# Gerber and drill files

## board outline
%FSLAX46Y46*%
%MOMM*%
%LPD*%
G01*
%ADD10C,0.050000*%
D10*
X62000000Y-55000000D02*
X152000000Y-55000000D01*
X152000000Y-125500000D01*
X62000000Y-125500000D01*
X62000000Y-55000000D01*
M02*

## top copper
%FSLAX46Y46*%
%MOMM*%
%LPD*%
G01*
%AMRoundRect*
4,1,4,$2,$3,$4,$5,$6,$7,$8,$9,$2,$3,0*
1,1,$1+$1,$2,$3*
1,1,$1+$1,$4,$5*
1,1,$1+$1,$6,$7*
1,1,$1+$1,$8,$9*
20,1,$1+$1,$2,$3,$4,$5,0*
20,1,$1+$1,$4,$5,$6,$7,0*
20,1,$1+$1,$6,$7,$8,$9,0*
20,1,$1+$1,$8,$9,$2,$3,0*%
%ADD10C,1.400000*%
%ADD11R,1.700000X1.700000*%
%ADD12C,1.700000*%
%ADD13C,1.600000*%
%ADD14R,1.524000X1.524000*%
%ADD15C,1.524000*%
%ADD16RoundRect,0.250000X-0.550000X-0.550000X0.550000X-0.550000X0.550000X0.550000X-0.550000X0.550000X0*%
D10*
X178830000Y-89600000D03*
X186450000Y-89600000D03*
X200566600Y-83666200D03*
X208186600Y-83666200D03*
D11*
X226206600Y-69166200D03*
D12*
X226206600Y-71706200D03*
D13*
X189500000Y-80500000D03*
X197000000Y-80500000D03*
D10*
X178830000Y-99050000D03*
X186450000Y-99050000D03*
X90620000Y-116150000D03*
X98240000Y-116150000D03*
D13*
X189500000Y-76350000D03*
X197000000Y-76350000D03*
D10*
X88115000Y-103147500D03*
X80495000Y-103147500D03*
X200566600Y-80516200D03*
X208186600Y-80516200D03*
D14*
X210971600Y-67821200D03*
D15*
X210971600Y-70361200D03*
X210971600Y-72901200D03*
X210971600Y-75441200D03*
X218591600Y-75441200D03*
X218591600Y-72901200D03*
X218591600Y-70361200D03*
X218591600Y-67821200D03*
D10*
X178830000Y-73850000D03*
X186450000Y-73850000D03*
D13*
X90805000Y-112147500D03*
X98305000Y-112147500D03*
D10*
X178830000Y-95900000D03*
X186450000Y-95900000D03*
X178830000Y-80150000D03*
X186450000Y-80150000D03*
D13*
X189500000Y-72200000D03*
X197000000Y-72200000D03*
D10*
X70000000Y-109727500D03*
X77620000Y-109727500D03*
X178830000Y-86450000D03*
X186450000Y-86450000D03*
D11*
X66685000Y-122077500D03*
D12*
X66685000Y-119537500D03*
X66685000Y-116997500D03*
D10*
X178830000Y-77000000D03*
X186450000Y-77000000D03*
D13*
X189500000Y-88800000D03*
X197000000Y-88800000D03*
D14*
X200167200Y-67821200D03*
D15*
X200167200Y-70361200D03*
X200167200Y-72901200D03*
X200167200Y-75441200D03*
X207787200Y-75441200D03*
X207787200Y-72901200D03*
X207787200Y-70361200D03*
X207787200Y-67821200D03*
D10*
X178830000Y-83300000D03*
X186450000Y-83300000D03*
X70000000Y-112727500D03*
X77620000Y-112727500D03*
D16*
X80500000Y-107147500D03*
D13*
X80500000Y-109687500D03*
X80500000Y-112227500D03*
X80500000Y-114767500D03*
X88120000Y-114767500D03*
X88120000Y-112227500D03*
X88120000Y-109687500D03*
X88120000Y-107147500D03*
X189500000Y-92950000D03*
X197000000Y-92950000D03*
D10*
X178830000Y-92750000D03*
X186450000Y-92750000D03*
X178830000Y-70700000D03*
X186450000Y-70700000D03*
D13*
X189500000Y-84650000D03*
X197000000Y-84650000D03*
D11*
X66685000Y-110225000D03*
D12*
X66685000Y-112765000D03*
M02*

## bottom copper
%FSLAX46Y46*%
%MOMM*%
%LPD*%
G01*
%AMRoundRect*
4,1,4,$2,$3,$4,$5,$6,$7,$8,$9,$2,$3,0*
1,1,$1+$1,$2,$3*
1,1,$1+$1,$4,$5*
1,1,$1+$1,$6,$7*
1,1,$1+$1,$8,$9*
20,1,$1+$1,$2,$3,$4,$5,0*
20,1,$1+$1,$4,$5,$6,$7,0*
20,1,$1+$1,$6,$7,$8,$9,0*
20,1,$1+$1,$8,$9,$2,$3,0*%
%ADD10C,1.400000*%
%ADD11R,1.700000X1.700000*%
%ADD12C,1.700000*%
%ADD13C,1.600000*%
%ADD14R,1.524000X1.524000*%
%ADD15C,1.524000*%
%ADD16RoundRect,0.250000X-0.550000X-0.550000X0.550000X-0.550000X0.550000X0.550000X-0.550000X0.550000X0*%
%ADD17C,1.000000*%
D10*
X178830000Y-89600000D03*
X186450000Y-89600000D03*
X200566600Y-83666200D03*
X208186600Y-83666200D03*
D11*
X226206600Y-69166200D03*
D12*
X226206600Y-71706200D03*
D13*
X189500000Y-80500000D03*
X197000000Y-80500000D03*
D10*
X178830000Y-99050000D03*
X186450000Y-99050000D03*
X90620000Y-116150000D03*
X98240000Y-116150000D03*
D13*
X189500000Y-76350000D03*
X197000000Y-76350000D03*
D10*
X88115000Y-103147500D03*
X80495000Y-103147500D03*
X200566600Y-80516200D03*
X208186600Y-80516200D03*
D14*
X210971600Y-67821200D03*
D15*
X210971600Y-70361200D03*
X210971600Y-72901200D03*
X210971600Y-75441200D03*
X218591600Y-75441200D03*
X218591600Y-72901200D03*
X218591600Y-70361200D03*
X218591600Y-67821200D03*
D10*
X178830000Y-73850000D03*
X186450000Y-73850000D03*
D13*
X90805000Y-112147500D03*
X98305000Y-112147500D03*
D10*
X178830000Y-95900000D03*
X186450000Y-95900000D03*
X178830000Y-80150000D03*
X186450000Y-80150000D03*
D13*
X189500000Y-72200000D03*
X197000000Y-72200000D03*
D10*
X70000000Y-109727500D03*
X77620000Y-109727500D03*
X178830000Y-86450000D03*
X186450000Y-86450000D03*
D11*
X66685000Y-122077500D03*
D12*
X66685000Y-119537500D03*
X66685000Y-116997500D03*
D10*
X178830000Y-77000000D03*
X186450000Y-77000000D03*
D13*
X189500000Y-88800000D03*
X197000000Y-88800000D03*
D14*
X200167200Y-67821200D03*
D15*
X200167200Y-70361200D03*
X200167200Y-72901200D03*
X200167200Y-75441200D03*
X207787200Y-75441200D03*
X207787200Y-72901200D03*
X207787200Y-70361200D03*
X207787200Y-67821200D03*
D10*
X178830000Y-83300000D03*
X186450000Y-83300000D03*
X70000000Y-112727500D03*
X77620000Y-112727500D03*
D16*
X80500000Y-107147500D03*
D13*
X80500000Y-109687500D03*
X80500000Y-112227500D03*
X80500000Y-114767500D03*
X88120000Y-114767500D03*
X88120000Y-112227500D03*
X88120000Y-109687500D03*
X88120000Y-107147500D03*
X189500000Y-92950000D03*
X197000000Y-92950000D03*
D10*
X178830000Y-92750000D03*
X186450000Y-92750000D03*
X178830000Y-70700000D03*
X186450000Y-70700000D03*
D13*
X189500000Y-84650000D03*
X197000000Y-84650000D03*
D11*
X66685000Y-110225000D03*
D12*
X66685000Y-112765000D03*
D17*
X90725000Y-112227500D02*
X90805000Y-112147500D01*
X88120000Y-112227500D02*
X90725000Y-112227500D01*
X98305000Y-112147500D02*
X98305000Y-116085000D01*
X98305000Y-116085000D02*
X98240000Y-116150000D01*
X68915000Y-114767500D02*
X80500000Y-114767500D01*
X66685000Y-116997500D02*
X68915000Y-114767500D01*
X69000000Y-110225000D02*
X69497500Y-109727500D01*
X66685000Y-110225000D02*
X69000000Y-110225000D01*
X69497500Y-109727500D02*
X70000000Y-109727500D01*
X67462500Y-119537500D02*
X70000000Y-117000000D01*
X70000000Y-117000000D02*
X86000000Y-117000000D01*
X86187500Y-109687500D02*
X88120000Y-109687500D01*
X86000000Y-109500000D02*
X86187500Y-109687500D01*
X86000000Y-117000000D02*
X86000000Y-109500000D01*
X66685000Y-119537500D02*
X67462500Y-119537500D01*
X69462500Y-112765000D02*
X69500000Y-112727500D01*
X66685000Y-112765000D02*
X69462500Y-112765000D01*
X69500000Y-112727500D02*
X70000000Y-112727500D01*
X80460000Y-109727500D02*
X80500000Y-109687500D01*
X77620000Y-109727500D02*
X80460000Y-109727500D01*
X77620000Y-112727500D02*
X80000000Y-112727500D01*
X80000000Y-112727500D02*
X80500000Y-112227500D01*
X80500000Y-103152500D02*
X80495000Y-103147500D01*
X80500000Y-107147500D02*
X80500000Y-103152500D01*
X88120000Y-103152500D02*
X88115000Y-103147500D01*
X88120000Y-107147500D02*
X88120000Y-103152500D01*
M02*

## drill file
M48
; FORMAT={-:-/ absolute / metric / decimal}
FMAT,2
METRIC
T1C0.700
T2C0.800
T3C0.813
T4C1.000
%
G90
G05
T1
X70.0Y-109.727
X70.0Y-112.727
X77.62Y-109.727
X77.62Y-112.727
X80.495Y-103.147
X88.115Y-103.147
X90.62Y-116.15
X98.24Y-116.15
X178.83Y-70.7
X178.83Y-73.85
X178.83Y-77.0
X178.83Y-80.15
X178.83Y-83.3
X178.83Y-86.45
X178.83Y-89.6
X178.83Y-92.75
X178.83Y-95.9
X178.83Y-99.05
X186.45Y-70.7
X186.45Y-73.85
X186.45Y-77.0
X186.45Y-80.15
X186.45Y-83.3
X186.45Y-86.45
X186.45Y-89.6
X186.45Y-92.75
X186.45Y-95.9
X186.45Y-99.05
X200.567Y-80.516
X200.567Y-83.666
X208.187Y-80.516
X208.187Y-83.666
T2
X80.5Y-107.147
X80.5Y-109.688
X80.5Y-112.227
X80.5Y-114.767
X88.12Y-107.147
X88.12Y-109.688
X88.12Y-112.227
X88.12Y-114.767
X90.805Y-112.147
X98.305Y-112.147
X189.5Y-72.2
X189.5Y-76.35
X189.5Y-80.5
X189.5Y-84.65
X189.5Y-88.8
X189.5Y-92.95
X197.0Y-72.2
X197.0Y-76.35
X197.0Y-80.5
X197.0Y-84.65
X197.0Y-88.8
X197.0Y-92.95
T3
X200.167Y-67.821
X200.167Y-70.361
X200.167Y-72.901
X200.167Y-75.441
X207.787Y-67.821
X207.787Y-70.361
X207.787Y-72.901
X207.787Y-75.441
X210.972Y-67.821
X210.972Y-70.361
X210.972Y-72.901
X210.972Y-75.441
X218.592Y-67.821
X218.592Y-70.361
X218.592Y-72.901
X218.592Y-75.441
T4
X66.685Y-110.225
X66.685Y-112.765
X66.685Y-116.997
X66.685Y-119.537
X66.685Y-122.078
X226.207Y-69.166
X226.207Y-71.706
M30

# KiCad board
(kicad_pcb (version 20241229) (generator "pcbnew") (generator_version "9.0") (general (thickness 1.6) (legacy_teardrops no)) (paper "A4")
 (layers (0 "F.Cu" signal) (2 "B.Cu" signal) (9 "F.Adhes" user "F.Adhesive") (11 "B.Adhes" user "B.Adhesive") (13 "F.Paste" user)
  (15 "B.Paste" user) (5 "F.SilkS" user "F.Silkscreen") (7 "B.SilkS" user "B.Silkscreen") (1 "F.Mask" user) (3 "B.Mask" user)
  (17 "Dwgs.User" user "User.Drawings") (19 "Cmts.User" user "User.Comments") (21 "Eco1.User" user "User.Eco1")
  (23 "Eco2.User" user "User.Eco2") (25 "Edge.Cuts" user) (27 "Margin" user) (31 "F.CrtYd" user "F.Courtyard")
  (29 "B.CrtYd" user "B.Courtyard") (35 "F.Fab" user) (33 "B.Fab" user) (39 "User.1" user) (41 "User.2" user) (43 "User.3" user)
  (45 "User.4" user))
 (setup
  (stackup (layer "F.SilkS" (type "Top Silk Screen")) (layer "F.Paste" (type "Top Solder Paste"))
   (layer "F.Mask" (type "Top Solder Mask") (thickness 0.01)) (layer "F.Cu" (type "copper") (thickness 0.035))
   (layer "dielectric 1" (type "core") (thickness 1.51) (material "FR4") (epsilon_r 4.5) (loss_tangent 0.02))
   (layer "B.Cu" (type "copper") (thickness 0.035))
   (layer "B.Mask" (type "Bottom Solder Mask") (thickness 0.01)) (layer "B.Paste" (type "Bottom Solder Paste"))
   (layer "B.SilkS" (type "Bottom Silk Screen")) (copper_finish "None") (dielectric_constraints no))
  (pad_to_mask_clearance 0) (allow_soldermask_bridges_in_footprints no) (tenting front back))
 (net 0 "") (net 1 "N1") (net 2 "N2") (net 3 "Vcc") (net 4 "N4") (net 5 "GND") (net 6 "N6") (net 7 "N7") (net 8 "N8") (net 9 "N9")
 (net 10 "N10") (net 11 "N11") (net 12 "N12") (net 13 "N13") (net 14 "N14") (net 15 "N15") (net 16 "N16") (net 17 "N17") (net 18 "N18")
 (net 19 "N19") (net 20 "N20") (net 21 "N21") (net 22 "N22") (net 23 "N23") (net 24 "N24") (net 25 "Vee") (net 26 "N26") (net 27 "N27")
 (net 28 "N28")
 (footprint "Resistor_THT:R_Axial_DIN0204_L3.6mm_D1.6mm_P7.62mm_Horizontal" (layer "F.Cu") (at 178.83 89.6)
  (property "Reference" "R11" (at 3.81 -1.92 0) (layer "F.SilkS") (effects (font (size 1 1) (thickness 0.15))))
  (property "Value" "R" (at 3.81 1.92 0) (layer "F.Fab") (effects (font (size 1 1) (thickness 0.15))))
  (pad "1" thru_hole circle (at 0 0) (size 1.4 1.4) (drill 0.7) (layers "*.Cu" "*.Mask") (remove_unused_layers no) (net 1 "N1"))
  (pad "2" thru_hole circle (at 7.62 0) (size 1.4 1.4) (drill 0.7) (layers "*.Cu" "*.Mask") (remove_unused_layers no) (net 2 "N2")))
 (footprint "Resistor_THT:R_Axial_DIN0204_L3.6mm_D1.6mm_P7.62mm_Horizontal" (layer "F.Cu") (at 200.5666 83.6662)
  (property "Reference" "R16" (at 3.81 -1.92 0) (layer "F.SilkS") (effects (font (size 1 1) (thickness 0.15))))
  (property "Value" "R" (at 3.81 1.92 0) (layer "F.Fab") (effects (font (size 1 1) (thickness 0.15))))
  (pad "1" thru_hole circle (at 0 0) (size 1.4 1.4) (drill 0.7) (layers "*.Cu" "*.Mask") (remove_unused_layers no) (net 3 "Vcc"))
  (pad "2" thru_hole circle (at 7.62 0) (size 1.4 1.4) (drill 0.7) (layers "*.Cu" "*.Mask") (remove_unused_layers no) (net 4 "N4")))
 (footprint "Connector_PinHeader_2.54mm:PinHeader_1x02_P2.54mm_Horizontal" (layer "F.Cu") (at 226.2066 69.1662)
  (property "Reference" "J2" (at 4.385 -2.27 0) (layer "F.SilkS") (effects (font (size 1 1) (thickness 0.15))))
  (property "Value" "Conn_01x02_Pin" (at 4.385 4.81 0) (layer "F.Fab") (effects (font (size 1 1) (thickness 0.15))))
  (pad "1" thru_hole rect (at 0 0) (size 1.7 1.7) (drill 1) (layers "*.Cu" "*.Mask") (remove_unused_layers no) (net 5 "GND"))
  (pad "2" thru_hole circle (at 0 2.54) (size 1.7 1.7) (drill 1) (layers "*.Cu" "*.Mask") (remove_unused_layers no) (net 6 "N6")))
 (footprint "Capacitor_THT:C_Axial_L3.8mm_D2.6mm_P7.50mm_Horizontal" (layer "F.Cu") (at 189.5 80.5)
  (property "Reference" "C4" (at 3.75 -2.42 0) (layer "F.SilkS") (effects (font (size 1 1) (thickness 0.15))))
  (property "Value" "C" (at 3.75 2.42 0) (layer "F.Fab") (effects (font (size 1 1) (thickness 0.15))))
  (pad "1" thru_hole circle (at 0 0) (size 1.6 1.6) (drill 0.8) (layers "*.Cu" "*.Mask") (remove_unused_layers no) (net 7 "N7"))
  (pad "2" thru_hole circle (at 7.5 0) (size 1.6 1.6) (drill 0.8) (layers "*.Cu" "*.Mask") (remove_unused_layers no) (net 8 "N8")))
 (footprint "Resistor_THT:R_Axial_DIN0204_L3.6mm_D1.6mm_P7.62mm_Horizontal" (layer "F.Cu") (at 178.83 99.05)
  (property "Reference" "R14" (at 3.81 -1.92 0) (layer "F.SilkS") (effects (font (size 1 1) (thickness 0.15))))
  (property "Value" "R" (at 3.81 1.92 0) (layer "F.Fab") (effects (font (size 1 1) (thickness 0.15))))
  (pad "1" thru_hole circle (at 0 0) (size 1.4 1.4) (drill 0.7) (layers "*.Cu" "*.Mask") (remove_unused_layers no) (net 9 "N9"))
  (pad "2" thru_hole circle (at 7.62 0) (size 1.4 1.4) (drill 0.7) (layers "*.Cu" "*.Mask") (remove_unused_layers no) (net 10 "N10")))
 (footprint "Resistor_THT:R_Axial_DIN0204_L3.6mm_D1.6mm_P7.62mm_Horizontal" (layer "F.Cu") (at 90.62 116.15)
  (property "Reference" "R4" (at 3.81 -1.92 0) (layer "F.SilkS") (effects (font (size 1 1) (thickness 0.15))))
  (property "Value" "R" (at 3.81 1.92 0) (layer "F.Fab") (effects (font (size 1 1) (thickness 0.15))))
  (pad "1" thru_hole circle (at 0 0) (size 1.4 1.4) (drill 0.7) (layers "*.Cu" "*.Mask") (remove_unused_layers no) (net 5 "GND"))
  (pad "2" thru_hole circle (at 7.62 0) (size 1.4 1.4) (drill 0.7) (layers "*.Cu" "*.Mask") (remove_unused_layers no) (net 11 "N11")))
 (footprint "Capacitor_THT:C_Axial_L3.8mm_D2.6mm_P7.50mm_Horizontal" (layer "F.Cu") (at 189.5 76.35)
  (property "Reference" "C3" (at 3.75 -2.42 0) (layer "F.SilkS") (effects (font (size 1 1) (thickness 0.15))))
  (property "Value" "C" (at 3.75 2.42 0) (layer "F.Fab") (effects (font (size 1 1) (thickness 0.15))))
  (pad "1" thru_hole circle (at 0 0) (size 1.6 1.6) (drill 0.8) (layers "*.Cu" "*.Mask") (remove_unused_layers no) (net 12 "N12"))
  (pad "2" thru_hole circle (at 7.5 0) (size 1.6 1.6) (drill 0.8) (layers "*.Cu" "*.Mask") (remove_unused_layers no) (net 5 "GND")))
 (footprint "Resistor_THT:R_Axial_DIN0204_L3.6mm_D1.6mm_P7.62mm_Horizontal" (layer "F.Cu") (at 88.115 103.1475 180)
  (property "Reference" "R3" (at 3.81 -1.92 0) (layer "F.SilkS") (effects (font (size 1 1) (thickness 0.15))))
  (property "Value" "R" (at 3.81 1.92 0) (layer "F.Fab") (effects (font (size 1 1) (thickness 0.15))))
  (pad "1" thru_hole circle (at 0 0 180) (size 1.4 1.4) (drill 0.7) (layers "*.Cu" "*.Mask") (remove_unused_layers no) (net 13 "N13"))
  (pad "2" thru_hole circle (at 7.62 0 180) (size 1.4 1.4) (drill 0.7) (layers "*.Cu" "*.Mask") (remove_unused_layers no) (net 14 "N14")))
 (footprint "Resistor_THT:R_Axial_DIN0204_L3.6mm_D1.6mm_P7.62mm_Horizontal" (layer "F.Cu") (at 200.5666 80.5162)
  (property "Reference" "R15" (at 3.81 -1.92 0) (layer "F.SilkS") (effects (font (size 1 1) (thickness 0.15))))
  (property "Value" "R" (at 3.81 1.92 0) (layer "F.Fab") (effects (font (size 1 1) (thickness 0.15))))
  (pad "1" thru_hole circle (at 0 0) (size 1.4 1.4) (drill 0.7) (layers "*.Cu" "*.Mask") (remove_unused_layers no) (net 5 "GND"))
  (pad "2" thru_hole circle (at 7.62 0) (size 1.4 1.4) (drill 0.7) (layers "*.Cu" "*.Mask") (remove_unused_layers no) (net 4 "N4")))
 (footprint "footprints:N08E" (layer "F.Cu") (at 218.5916 75.4412)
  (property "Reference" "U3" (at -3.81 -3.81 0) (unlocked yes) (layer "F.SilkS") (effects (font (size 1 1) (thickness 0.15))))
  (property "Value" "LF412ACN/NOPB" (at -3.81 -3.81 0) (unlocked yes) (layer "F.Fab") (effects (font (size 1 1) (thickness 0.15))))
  (pad "1" thru_hole rect (at -7.62 -7.62) (size 1.524 1.524) (drill 0.8128) (layers "*.Cu" "*.Mask") (remove_unused_layers no)
   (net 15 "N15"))
  (pad "2" thru_hole circle (at -7.62 -5.08) (size 1.524 1.524) (drill 0.8128) (layers "*.Cu" "*.Mask") (remove_unused_layers no)
   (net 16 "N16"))
  (pad "3" thru_hole circle (at -7.62 -2.54) (size 1.524 1.524) (drill 0.8128) (layers "*.Cu" "*.Mask") (remove_unused_layers no)
   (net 5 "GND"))
  (pad "4" thru_hole circle (at -7.62 0) (size 1.524 1.524) (drill 0.8128) (layers "*.Cu" "*.Mask") (remove_unused_layers no))
  (pad "5" thru_hole circle (at 0 0) (size 1.524 1.524) (drill 0.8128) (layers "*.Cu" "*.Mask") (remove_unused_layers no) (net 4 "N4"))
  (pad "6" thru_hole circle (at 0 -2.54) (size 1.524 1.524) (drill 0.8128) (layers "*.Cu" "*.Mask") (remove_unused_layers no) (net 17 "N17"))
  (pad "7" thru_hole circle (at 0 -5.08) (size 1.524 1.524) (drill 0.8128) (layers "*.Cu" "*.Mask") (remove_unused_layers no) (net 6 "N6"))
  (pad "8" thru_hole circle (at 0 -7.62) (size 1.524 1.524) (drill 0.8128) (layers "*.Cu" "*.Mask") (remove_unused_layers no)))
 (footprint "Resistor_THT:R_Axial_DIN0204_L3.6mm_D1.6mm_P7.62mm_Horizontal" (layer "F.Cu") (at 178.83 73.85)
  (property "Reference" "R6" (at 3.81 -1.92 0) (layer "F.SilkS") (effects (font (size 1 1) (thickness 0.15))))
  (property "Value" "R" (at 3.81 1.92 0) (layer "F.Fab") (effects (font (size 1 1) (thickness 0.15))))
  (pad "1" thru_hole circle (at 0 0) (size 1.4 1.4) (drill 0.7) (layers "*.Cu" "*.Mask") (remove_unused_layers no) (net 12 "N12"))
  (pad "2" thru_hole circle (at 7.62 0) (size 1.4 1.4) (drill 0.7) (layers "*.Cu" "*.Mask") (remove_unused_layers no) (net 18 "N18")))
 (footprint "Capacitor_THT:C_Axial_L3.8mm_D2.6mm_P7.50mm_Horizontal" (layer "F.Cu") (at 90.805 112.1475)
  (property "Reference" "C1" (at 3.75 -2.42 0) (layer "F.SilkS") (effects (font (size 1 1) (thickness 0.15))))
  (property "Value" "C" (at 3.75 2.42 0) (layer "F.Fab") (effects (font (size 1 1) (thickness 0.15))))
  (pad "1" thru_hole circle (at 0 0) (size 1.6 1.6) (drill 0.8) (layers "*.Cu" "*.Mask") (remove_unused_layers no) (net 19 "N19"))
  (pad "2" thru_hole circle (at 7.5 0) (size 1.6 1.6) (drill 0.8) (layers "*.Cu" "*.Mask") (remove_unused_layers no) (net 11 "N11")))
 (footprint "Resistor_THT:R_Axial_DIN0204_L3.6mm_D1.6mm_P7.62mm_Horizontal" (layer "F.Cu") (at 178.83 95.9)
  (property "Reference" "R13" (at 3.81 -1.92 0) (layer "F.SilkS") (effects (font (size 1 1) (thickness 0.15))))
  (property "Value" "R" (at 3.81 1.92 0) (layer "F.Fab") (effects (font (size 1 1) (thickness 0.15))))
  (pad "1" thru_hole circle (at 0 0) (size 1.4 1.4) (drill 0.7) (layers "*.Cu" "*.Mask") (remove_unused_layers no) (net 5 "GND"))
  (pad "2" thru_hole circle (at 7.62 0) (size 1.4 1.4) (drill 0.7) (layers "*.Cu" "*.Mask") (remove_unused_layers no) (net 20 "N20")))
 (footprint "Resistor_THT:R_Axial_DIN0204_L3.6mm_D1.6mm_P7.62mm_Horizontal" (layer "F.Cu") (at 178.83 80.15)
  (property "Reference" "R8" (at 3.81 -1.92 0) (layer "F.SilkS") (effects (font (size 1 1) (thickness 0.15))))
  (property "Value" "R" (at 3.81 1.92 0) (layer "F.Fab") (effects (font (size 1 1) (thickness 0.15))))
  (pad "1" thru_hole circle (at 0 0) (size 1.4 1.4) (drill 0.7) (layers "*.Cu" "*.Mask") (remove_unused_layers no) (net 5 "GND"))
  (pad "2" thru_hole circle (at 7.62 0) (size 1.4 1.4) (drill 0.7) (layers "*.Cu" "*.Mask") (remove_unused_layers no) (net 7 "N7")))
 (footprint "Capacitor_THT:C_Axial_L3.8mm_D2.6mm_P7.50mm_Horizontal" (layer "F.Cu") (at 189.5 72.2)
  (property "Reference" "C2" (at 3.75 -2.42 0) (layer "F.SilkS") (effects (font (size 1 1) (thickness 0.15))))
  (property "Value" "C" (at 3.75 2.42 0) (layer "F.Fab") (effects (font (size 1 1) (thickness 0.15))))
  (pad "1" thru_hole circle (at 0 0) (size 1.6 1.6) (drill 0.8) (layers "*.Cu" "*.Mask") (remove_unused_layers no) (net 12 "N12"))
  (pad "2" thru_hole circle (at 7.5 0) (size 1.6 1.6) (drill 0.8) (layers "*.Cu" "*.Mask") (remove_unused_layers no) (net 5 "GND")))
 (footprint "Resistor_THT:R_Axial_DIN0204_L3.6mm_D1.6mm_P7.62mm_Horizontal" (layer "F.Cu") (at 70 109.7275)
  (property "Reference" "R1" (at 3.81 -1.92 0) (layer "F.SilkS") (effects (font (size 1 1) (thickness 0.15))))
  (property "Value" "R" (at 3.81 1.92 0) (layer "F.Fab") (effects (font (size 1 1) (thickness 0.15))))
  (pad "1" thru_hole circle (at 0 0) (size 1.4 1.4) (drill 0.7) (layers "*.Cu" "*.Mask") (remove_unused_layers no) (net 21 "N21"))
  (pad "2" thru_hole circle (at 7.62 0) (size 1.4 1.4) (drill 0.7) (layers "*.Cu" "*.Mask") (remove_unused_layers no) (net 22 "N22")))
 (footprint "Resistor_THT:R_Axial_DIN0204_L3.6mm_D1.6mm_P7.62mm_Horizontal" (layer "F.Cu") (at 178.83 86.45)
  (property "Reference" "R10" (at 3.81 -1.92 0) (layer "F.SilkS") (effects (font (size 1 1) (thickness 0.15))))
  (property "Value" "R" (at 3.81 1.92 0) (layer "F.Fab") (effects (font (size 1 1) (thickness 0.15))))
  (pad "1" thru_hole circle (at 0 0) (size 1.4 1.4) (drill 0.7) (layers "*.Cu" "*.Mask") (remove_unused_layers no) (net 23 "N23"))
  (pad "2" thru_hole circle (at 7.62 0) (size 1.4 1.4) (drill 0.7) (layers "*.Cu" "*.Mask") (remove_unused_layers no) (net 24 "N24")))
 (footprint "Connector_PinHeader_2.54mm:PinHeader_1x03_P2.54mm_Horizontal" (layer "F.Cu") (at 66.685 122.0775 180)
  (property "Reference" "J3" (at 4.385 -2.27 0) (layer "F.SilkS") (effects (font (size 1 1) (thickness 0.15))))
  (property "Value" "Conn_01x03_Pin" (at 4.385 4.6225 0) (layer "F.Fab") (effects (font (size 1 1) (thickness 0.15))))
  (pad "1" thru_hole rect (at 0 0 180) (size 1.7 1.7) (drill 1) (layers "*.Cu" "*.Mask") (remove_unused_layers no) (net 5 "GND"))
  (pad "2" thru_hole circle (at 0 2.54 180) (size 1.7 1.7) (drill 1) (layers "*.Cu" "*.Mask") (remove_unused_layers no) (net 3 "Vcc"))
  (pad "3" thru_hole circle (at 0 5.08 180) (size 1.7 1.7) (drill 1) (layers "*.Cu" "*.Mask") (remove_unused_layers no) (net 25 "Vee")))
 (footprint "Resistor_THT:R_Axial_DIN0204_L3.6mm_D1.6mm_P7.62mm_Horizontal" (layer "F.Cu") (at 178.83 77)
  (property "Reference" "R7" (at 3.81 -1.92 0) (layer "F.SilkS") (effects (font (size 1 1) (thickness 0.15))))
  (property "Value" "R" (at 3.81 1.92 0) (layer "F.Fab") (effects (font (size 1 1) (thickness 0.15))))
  (pad "1" thru_hole circle (at 0 0) (size 1.4 1.4) (drill 0.7) (layers "*.Cu" "*.Mask") (remove_unused_layers no) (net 5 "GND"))
  (pad "2" thru_hole circle (at 7.62 0) (size 1.4 1.4) (drill 0.7) (layers "*.Cu" "*.Mask") (remove_unused_layers no) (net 7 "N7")))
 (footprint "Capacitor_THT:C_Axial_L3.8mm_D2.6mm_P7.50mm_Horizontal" (layer "F.Cu") (at 189.5 88.8)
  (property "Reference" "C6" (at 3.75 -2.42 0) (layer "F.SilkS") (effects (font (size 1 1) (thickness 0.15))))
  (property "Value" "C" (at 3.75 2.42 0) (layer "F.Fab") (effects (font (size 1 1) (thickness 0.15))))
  (pad "1" thru_hole circle (at 0 0) (size 1.6 1.6) (drill 0.8) (layers "*.Cu" "*.Mask") (remove_unused_layers no) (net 23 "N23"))
  (pad "2" thru_hole circle (at 7.5 0) (size 1.6 1.6) (drill 0.8) (layers "*.Cu" "*.Mask") (remove_unused_layers no) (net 24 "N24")))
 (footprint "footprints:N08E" (layer "F.Cu") (at 207.7872 75.4412)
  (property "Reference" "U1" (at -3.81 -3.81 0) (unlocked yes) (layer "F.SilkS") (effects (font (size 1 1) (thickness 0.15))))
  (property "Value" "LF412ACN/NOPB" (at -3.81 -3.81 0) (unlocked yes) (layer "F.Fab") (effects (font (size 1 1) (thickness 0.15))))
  (pad "1" thru_hole rect (at -7.62 -7.62) (size 1.524 1.524) (drill 0.8128) (layers "*.Cu" "*.Mask") (remove_unused_layers no) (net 8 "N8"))
  (pad "2" thru_hole circle (at -7.62 -5.08) (size 1.524 1.524) (drill 0.8128) (layers "*.Cu" "*.Mask") (remove_unused_layers no)
   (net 8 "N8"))
  (pad "3" thru_hole circle (at -7.62 -2.54) (size 1.524 1.524) (drill 0.8128) (layers "*.Cu" "*.Mask") (remove_unused_layers no)
   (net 11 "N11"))
  (pad "4" thru_hole circle (at -7.62 0) (size 1.524 1.524) (drill 0.8128) (layers "*.Cu" "*.Mask") (remove_unused_layers no))
  (pad "5" thru_hole circle (at 0 0) (size 1.524 1.524) (drill 0.8128) (layers "*.Cu" "*.Mask") (remove_unused_layers no) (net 18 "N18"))
  (pad "6" thru_hole circle (at 0 -2.54) (size 1.524 1.524) (drill 0.8128) (layers "*.Cu" "*.Mask") (remove_unused_layers no) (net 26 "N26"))
  (pad "7" thru_hole circle (at 0 -5.08) (size 1.524 1.524) (drill 0.8128) (layers "*.Cu" "*.Mask") (remove_unused_layers no) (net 26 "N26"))
  (pad "8" thru_hole circle (at 0 -7.62) (size 1.524 1.524) (drill 0.8128) (layers "*.Cu" "*.Mask") (remove_unused_layers no)))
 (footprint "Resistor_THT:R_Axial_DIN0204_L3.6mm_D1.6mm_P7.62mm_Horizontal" (layer "F.Cu") (at 178.83 83.3)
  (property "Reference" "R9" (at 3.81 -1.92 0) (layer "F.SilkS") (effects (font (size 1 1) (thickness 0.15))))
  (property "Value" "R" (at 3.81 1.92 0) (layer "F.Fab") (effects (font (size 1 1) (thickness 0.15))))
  (pad "1" thru_hole circle (at 0 0) (size 1.4 1.4) (drill 0.7) (layers "*.Cu" "*.Mask") (remove_unused_layers no) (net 26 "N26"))
  (pad "2" thru_hole circle (at 7.62 0) (size 1.4 1.4) (drill 0.7) (layers "*.Cu" "*.Mask") (remove_unused_layers no) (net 16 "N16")))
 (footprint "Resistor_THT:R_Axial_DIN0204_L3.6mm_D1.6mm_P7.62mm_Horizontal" (layer "F.Cu") (at 70 112.7275)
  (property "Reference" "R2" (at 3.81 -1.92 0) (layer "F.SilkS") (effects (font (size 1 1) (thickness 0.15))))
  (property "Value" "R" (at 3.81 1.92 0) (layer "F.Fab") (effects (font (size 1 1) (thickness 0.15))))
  (pad "1" thru_hole circle (at 0 0) (size 1.4 1.4) (drill 0.7) (layers "*.Cu" "*.Mask") (remove_unused_layers no) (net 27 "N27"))
  (pad "2" thru_hole circle (at 7.62 0) (size 1.4 1.4) (drill 0.7) (layers "*.Cu" "*.Mask") (remove_unused_layers no) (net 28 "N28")))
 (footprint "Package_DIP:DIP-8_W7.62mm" (layer "F.Cu") (at 80.5 107.1475)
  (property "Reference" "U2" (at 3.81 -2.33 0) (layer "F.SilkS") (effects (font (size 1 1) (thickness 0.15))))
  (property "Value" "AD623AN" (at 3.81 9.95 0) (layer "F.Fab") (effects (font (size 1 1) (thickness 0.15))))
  (pad "1" thru_hole roundrect (at 0 0) (size 1.6 1.6) (drill 0.8) (layers "*.Cu" "*.Mask") (remove_unused_layers no)
   (roundrect_rratio 0.15625) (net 14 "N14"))
  (pad "2" thru_hole circle (at 0 2.54) (size 1.6 1.6) (drill 0.8) (layers "*.Cu" "*.Mask") (remove_unused_layers no) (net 22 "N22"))
  (pad "3" thru_hole circle (at 0 5.08) (size 1.6 1.6) (drill 0.8) (layers "*.Cu" "*.Mask") (remove_unused_layers no) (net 28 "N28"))
  (pad "4" thru_hole circle (at 0 7.62) (size 1.6 1.6) (drill 0.8) (layers "*.Cu" "*.Mask") (remove_unused_layers no) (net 25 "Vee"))
  (pad "5" thru_hole circle (at 7.62 7.62) (size 1.6 1.6) (drill 0.8) (layers "*.Cu" "*.Mask") (remove_unused_layers no) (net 5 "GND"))
  (pad "6" thru_hole circle (at 7.62 5.08) (size 1.6 1.6) (drill 0.8) (layers "*.Cu" "*.Mask") (remove_unused_layers no) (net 19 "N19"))
  (pad "7" thru_hole circle (at 7.62 2.54) (size 1.6 1.6) (drill 0.8) (layers "*.Cu" "*.Mask") (remove_unused_layers no) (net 3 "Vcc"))
  (pad "8" thru_hole circle (at 7.62 0) (size 1.6 1.6) (drill 0.8) (layers "*.Cu" "*.Mask") (remove_unused_layers no) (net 13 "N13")))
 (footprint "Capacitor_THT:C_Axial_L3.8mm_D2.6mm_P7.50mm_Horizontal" (layer "F.Cu") (at 189.5 92.95)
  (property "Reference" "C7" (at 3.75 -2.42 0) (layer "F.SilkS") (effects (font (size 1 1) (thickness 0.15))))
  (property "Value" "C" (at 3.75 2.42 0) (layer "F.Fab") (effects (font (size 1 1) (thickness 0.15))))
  (pad "1" thru_hole circle (at 0 0) (size 1.6 1.6) (drill 0.8) (layers "*.Cu" "*.Mask") (remove_unused_layers no) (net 15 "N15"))
  (pad "2" thru_hole circle (at 7.5 0) (size 1.6 1.6) (drill 0.8) (layers "*.Cu" "*.Mask") (remove_unused_layers no) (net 1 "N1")))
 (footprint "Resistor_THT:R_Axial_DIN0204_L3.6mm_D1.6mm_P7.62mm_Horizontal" (layer "F.Cu") (at 178.83 92.75)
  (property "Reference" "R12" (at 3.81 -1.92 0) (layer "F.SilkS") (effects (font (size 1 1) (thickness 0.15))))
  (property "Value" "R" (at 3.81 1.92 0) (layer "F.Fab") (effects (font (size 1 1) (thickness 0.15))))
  (pad "1" thru_hole circle (at 0 0) (size 1.4 1.4) (drill 0.7) (layers "*.Cu" "*.Mask") (remove_unused_layers no) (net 2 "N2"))
  (pad "2" thru_hole circle (at 7.62 0) (size 1.4 1.4) (drill 0.7) (layers "*.Cu" "*.Mask") (remove_unused_layers no) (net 17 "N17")))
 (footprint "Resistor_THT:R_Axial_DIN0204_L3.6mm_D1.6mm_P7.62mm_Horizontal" (layer "F.Cu") (at 178.83 70.7)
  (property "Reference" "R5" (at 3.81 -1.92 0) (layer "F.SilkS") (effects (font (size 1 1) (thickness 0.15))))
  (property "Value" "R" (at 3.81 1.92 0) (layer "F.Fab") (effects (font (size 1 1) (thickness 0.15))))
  (pad "1" thru_hole circle (at 0 0) (size 1.4 1.4) (drill 0.7) (layers "*.Cu" "*.Mask") (remove_unused_layers no) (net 8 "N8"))
  (pad "2" thru_hole circle (at 7.62 0) (size 1.4 1.4) (drill 0.7) (layers "*.Cu" "*.Mask") (remove_unused_layers no) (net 12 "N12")))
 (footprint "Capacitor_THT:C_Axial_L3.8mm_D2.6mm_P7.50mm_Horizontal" (layer "F.Cu") (at 189.5 84.65)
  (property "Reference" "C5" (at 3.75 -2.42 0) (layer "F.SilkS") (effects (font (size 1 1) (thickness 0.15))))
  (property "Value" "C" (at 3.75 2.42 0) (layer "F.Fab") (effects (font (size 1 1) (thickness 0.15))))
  (pad "1" thru_hole circle (at 0 0) (size 1.6 1.6) (drill 0.8) (layers "*.Cu" "*.Mask") (remove_unused_layers no) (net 18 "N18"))
  (pad "2" thru_hole circle (at 7.5 0) (size 1.6 1.6) (drill 0.8) (layers "*.Cu" "*.Mask") (remove_unused_layers no) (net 7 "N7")))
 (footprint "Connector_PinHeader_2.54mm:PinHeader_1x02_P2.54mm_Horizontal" (layer "B.Cu") (at 66.685 110.225 180)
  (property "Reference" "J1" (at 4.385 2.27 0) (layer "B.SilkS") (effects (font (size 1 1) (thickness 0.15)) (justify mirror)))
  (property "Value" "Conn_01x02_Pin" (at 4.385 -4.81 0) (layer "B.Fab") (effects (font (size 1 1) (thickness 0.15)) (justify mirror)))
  (pad "1" thru_hole rect (at 0 0 180) (size 1.7 1.7) (drill 1) (layers "*.Cu" "*.Mask") (remove_unused_layers no) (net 21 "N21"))
  (pad "2" thru_hole circle (at 0 -2.54 180) (size 1.7 1.7) (drill 1) (layers "*.Cu" "*.Mask") (remove_unused_layers no) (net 27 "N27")))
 (gr_rect (start 62 55) (end 152 125.5) (stroke (width 0.05) (type default)) (fill no) (layer "Edge.Cuts"))
 (segment (start 90.725 112.2275) (end 90.805 112.1475) (width 1) (layer "B.Cu") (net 19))
 (segment (start 88.12 112.2275) (end 90.725 112.2275) (width 1) (layer "B.Cu") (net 19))
 (segment (start 98.305 112.1475) (end 98.305 116.085) (width 1) (layer "B.Cu") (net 11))
 (segment (start 98.305 116.085) (end 98.24 116.15) (width 1) (layer "B.Cu") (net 11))
 (segment (start 68.915 114.7675) (end 80.5 114.7675) (width 1) (layer "B.Cu") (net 25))
 (segment (start 66.685 116.9975) (end 68.915 114.7675) (width 1) (layer "B.Cu") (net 25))
 (segment (start 69 110.225) (end 69.4975 109.7275) (width 1) (layer "B.Cu") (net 21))
 (segment (start 66.685 110.225) (end 69 110.225) (width 1) (layer "B.Cu") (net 21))
 (segment (start 69.4975 109.7275) (end 70 109.7275) (width 1) (layer "B.Cu") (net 21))
 (segment (start 67.4625 119.5375) (end 70 117) (width 1) (layer "B.Cu") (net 3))
 (segment (start 70 117) (end 86 117) (width 1) (layer "B.Cu") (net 3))
 (segment (start 86.1875 109.6875) (end 88.12 109.6875) (width 1) (layer "B.Cu") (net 3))
 (segment (start 86 109.5) (end 86.1875 109.6875) (width 1) (layer "B.Cu") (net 3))
 (segment (start 86 117) (end 86 109.5) (width 1) (layer "B.Cu") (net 3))
 (segment (start 66.685 119.5375) (end 67.4625 119.5375) (width 1) (layer "B.Cu") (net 3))
 (segment (start 69.4625 112.765) (end 69.5 112.7275) (width 1) (layer "B.Cu") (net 27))
 (segment (start 66.685 112.765) (end 69.4625 112.765) (width 1) (layer "B.Cu") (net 27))
 (segment (start 69.5 112.7275) (end 70 112.7275) (width 1) (layer "B.Cu") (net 27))
 (segment (start 80.46 109.7275) (end 80.5 109.6875) (width 1) (layer "B.Cu") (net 22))
 (segment (start 77.62 109.7275) (end 80.46 109.7275) (width 1) (layer "B.Cu") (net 22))
 (segment (start 77.62 112.7275) (end 80 112.7275) (width 1) (layer "B.Cu") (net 28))
 (segment (start 80 112.7275) (end 80.5 112.2275) (width 1) (layer "B.Cu") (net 28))
 (segment (start 80.5 103.1525) (end 80.495 103.1475) (width 1) (layer "B.Cu") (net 14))
 (segment (start 80.5 107.1475) (end 80.5 103.1525) (width 1) (layer "B.Cu") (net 14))
 (segment (start 88.12 103.1525) (end 88.115 103.1475) (width 1) (layer "B.Cu") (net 13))
 (segment (start 88.12 107.1475) (end 88.12 103.1525) (width 1) (layer "B.Cu") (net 13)))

